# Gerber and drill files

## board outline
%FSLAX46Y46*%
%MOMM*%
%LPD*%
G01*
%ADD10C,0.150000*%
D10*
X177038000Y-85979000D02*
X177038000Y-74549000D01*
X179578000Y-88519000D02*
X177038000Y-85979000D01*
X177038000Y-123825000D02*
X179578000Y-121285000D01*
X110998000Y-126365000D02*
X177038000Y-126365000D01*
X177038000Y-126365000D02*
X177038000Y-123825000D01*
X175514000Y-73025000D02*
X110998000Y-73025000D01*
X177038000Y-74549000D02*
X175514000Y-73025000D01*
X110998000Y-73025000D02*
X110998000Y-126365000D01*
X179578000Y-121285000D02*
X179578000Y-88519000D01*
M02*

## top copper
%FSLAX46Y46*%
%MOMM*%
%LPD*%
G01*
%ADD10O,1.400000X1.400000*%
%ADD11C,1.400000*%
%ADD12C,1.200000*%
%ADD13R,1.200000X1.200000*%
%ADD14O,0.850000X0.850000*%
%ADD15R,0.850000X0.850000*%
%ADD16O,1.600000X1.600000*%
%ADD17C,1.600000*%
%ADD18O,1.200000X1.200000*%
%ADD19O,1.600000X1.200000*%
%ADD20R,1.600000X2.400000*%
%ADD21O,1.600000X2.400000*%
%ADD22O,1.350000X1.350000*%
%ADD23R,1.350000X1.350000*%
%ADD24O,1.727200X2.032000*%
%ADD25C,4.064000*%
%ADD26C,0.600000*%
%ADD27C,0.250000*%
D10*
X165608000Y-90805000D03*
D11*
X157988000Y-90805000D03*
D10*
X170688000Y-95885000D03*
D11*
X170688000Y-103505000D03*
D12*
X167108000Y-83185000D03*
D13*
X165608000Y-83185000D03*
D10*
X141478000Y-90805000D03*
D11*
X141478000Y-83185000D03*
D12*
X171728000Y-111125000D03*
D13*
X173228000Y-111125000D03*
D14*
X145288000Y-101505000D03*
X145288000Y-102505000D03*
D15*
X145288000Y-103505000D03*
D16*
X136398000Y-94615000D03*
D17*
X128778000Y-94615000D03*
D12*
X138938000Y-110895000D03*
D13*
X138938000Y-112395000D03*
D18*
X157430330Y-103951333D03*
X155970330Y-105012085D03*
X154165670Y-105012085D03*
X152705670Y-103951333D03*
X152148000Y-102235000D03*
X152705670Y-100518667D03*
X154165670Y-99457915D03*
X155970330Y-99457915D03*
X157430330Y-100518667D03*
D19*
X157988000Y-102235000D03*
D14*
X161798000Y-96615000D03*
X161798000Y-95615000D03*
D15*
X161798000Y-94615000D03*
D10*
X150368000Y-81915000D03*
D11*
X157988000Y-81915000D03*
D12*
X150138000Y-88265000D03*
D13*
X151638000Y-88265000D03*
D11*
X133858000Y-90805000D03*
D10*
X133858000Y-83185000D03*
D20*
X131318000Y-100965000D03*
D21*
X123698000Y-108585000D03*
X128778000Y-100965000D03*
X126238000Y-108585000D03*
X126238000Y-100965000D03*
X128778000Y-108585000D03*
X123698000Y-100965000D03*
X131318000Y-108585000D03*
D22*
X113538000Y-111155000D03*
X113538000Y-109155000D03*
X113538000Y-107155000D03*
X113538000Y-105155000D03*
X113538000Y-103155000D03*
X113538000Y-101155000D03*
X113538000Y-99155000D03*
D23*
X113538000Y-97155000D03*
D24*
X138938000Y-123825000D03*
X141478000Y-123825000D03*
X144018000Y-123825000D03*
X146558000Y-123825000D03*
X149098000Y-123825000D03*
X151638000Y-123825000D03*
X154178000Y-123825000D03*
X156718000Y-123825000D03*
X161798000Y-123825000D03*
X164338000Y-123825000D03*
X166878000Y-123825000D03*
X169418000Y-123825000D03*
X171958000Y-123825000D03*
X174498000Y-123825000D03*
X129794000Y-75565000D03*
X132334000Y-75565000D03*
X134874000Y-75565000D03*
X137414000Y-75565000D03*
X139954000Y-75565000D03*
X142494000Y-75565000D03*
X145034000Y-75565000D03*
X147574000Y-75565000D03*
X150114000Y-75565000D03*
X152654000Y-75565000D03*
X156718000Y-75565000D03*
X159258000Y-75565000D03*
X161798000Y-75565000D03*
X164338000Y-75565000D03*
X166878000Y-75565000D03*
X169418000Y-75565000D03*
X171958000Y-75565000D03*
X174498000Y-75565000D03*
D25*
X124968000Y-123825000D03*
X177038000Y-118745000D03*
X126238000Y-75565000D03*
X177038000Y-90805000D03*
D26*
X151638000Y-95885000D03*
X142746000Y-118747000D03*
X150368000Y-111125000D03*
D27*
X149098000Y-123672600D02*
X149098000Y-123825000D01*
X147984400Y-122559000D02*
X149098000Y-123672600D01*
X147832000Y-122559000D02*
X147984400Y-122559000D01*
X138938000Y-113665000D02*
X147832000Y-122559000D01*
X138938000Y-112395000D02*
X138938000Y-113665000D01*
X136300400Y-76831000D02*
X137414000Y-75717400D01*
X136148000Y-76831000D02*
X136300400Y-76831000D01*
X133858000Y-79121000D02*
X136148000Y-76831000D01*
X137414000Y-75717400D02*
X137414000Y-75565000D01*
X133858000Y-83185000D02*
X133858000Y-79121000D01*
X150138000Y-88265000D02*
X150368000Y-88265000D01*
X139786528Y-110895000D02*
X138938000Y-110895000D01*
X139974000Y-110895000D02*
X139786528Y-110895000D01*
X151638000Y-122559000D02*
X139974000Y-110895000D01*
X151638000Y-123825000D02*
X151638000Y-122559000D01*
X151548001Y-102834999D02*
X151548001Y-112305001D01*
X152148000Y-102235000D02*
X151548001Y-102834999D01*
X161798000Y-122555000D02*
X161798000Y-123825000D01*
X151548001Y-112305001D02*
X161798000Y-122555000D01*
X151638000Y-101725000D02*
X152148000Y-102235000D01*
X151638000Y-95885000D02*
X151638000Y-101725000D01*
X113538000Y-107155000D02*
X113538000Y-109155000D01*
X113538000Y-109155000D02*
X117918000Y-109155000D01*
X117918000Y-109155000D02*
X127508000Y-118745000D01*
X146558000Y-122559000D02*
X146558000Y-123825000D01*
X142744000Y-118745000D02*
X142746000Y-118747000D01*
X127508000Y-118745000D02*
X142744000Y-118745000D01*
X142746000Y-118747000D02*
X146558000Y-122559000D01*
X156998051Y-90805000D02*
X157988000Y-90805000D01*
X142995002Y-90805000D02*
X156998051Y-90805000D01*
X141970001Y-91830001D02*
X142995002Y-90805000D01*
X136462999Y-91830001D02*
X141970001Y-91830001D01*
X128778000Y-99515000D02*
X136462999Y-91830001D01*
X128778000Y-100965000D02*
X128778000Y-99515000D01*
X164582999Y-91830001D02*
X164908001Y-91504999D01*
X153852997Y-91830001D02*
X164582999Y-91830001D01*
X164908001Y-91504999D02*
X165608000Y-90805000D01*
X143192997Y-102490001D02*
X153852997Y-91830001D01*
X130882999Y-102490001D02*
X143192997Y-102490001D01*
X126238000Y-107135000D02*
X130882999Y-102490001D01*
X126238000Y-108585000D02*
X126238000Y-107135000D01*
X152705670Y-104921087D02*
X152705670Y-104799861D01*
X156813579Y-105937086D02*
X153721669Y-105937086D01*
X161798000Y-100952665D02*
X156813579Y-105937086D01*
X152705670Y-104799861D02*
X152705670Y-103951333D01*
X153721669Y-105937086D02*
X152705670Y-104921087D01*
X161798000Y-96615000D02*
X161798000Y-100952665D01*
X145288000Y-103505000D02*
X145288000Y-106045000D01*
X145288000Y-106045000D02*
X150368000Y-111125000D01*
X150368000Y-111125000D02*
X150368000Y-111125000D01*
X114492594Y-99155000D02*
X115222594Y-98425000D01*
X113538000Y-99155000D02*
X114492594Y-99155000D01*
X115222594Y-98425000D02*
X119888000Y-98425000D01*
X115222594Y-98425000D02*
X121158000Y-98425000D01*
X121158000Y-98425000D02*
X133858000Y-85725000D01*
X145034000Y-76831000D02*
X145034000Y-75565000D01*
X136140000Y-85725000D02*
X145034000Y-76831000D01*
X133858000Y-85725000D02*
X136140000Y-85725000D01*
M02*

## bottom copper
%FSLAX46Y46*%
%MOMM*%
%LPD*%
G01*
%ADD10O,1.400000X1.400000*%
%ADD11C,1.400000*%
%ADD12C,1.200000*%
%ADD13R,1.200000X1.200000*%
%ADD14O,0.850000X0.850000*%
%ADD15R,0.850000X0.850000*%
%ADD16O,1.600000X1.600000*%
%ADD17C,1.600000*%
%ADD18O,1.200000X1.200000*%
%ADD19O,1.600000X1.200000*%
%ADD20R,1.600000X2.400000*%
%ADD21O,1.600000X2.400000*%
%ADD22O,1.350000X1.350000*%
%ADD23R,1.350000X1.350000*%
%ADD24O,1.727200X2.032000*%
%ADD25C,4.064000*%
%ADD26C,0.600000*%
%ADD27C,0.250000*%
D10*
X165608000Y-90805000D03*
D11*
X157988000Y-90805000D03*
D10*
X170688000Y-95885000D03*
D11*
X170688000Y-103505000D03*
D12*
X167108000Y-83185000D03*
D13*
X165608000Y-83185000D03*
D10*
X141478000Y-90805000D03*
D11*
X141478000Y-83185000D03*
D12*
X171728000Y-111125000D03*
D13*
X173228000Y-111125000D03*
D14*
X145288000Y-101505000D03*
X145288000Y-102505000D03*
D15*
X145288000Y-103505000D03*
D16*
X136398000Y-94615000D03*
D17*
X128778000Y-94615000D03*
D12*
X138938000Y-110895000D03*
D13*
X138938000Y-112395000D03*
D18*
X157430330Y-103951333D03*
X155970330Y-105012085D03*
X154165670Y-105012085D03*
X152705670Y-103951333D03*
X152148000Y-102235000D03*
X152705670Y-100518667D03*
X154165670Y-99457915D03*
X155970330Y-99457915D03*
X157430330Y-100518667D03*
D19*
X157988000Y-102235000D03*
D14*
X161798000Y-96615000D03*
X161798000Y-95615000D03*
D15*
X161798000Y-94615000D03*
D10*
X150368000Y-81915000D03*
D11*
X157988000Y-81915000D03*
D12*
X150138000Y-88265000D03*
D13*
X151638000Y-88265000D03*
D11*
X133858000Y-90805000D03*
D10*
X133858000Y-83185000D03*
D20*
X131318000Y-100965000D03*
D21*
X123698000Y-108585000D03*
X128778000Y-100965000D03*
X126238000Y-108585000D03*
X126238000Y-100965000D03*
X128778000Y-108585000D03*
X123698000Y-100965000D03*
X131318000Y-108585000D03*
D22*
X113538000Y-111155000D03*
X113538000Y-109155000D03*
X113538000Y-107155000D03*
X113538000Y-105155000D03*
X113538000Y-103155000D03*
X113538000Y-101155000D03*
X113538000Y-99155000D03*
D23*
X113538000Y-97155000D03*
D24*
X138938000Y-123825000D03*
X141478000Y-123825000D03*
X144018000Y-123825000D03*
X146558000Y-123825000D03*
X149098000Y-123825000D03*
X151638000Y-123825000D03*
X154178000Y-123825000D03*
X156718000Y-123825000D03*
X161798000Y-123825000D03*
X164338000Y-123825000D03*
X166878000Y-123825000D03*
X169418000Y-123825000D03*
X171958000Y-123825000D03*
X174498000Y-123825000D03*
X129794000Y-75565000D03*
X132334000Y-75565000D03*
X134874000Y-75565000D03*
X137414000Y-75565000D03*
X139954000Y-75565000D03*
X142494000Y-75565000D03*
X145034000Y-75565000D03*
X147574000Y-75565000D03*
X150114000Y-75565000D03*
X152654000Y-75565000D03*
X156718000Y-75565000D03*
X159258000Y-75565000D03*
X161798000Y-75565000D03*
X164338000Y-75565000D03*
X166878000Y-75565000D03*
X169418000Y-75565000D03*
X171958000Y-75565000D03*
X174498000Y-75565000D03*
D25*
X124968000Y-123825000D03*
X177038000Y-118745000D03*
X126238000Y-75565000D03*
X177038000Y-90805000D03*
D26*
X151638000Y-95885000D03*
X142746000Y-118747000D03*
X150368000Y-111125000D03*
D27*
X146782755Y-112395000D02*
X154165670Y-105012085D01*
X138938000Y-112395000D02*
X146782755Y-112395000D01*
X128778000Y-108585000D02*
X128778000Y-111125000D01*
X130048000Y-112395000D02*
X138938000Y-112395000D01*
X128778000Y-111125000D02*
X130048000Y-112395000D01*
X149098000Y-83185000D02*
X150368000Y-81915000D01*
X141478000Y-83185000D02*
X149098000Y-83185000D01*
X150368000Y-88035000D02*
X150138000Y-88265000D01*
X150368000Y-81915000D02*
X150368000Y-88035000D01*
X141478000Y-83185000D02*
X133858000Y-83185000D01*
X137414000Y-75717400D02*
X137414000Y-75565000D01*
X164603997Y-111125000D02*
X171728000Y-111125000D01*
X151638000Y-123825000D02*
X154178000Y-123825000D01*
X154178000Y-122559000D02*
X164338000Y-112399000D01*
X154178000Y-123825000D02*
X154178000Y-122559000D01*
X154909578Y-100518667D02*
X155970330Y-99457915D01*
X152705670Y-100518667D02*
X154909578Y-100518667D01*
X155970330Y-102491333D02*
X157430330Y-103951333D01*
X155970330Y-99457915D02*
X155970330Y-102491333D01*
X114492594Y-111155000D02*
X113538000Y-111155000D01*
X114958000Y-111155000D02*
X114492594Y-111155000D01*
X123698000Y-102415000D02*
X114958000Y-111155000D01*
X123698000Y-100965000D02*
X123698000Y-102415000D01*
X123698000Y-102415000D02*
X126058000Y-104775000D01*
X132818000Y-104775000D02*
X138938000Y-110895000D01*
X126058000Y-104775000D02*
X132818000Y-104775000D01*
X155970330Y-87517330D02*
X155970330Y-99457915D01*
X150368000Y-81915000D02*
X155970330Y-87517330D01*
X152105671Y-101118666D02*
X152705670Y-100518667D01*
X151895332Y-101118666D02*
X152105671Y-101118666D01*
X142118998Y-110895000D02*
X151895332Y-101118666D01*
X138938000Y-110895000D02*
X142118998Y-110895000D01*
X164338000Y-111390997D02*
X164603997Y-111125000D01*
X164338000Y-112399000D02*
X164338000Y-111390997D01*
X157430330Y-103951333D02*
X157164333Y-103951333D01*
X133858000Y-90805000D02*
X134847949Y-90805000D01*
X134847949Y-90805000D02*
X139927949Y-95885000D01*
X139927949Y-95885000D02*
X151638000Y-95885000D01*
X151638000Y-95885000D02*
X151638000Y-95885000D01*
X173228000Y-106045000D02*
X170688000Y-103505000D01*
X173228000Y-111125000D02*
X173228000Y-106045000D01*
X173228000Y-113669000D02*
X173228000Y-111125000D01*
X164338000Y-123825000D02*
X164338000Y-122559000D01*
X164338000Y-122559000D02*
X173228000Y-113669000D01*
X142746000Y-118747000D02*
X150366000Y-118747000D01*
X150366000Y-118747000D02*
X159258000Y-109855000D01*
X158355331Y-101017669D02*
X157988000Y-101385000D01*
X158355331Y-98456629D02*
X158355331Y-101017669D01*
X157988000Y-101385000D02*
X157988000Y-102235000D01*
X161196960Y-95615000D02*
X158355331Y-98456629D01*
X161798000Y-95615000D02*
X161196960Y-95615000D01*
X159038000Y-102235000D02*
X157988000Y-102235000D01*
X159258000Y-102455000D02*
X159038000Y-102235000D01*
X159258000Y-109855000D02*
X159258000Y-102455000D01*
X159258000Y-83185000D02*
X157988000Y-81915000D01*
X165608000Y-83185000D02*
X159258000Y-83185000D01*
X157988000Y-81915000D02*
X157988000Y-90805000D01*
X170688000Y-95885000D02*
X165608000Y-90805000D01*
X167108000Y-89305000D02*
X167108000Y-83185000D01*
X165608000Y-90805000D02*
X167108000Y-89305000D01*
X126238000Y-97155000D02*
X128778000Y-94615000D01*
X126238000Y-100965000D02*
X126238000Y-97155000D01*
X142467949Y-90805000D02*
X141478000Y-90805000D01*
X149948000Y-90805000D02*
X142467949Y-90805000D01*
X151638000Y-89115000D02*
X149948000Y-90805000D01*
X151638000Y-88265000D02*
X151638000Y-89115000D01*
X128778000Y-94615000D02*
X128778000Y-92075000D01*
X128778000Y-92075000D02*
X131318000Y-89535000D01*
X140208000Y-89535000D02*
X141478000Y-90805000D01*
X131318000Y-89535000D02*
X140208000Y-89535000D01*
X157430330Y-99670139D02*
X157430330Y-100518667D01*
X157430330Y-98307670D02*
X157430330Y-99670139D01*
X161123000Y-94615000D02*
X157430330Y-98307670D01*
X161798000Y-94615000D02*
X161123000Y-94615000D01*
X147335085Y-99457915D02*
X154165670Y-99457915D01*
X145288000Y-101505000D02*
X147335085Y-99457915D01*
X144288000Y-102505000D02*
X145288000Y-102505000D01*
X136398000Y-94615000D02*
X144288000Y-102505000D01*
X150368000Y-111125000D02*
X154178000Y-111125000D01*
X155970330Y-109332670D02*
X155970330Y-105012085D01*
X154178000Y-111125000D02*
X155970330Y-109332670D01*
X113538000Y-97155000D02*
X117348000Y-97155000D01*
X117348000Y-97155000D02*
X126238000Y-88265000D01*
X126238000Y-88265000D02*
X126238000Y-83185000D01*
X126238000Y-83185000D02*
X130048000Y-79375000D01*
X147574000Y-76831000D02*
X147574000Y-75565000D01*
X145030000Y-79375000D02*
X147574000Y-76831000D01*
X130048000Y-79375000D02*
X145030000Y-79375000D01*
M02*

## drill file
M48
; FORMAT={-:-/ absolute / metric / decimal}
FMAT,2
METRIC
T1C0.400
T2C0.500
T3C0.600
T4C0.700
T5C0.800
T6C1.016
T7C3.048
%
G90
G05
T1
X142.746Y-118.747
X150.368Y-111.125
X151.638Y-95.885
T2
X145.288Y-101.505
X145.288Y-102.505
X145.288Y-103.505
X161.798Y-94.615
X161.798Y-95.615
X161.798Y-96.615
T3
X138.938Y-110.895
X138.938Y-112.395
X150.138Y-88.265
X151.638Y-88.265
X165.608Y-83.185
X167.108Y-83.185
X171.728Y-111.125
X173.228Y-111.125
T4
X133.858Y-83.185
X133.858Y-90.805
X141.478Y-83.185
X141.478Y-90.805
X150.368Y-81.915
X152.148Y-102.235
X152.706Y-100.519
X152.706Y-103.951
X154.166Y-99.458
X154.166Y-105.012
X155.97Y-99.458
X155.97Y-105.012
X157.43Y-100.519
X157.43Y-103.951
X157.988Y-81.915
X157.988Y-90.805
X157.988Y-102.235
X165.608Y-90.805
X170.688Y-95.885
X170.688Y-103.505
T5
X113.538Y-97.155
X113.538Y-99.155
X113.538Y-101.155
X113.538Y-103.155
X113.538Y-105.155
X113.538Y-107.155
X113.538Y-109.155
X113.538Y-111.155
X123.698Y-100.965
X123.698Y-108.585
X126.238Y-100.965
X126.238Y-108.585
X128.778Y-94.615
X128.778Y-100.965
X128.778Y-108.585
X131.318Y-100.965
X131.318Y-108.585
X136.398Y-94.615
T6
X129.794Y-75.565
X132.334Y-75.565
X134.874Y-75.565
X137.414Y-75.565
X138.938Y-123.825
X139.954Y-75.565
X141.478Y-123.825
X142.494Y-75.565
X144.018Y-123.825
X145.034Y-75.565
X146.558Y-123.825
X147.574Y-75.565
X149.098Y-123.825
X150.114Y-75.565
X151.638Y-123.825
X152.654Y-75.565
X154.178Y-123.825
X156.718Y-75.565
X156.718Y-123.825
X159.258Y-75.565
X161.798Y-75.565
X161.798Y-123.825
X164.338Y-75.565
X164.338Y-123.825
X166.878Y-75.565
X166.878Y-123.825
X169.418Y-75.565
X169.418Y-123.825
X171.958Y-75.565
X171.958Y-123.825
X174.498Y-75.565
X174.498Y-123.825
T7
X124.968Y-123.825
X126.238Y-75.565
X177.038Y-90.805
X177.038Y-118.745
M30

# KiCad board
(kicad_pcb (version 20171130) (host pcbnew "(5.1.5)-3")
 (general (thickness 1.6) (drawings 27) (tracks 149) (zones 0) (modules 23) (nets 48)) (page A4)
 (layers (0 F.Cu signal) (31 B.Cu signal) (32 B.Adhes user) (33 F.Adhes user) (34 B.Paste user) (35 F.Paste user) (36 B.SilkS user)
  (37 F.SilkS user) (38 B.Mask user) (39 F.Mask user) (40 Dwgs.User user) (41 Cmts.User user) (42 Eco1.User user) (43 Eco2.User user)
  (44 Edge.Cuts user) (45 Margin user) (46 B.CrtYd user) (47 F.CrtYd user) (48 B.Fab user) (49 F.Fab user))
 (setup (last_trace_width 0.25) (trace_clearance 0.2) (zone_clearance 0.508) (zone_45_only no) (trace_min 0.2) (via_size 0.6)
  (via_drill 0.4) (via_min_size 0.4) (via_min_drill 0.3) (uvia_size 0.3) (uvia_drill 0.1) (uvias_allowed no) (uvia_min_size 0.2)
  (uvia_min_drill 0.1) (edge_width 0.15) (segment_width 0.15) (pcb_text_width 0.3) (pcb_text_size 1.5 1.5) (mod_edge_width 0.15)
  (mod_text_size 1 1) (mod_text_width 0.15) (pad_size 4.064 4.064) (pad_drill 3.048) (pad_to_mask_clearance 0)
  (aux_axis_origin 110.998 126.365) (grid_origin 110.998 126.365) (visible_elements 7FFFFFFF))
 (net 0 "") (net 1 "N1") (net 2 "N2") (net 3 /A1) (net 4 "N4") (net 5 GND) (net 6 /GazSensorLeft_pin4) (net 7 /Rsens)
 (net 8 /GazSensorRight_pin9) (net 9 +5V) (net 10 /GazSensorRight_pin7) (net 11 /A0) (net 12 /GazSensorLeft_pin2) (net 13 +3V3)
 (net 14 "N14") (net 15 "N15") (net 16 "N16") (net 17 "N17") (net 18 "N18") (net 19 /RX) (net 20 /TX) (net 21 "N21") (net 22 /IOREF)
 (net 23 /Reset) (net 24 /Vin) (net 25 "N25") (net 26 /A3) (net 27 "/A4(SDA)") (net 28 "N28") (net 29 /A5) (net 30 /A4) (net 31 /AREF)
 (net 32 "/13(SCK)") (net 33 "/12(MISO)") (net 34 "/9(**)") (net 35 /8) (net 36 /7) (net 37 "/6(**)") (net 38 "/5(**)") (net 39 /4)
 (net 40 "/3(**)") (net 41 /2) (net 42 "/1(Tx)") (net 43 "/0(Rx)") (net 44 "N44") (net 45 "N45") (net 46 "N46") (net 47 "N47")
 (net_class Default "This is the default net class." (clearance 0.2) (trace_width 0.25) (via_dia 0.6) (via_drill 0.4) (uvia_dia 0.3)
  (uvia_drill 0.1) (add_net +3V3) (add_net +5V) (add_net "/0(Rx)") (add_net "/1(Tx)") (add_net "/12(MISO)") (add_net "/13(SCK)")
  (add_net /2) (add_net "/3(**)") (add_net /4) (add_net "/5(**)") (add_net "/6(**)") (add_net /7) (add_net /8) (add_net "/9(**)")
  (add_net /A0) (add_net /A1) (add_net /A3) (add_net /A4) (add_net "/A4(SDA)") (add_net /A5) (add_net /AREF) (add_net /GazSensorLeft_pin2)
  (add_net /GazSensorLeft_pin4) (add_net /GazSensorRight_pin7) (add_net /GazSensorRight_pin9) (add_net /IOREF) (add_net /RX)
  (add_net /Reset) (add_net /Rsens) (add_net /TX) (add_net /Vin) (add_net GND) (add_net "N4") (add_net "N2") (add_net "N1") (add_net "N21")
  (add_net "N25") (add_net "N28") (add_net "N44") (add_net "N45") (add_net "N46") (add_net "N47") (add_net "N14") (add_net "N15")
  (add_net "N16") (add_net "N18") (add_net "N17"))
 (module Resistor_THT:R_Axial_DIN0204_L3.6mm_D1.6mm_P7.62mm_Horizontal (layer F.Cu) (at 157.988 90.805)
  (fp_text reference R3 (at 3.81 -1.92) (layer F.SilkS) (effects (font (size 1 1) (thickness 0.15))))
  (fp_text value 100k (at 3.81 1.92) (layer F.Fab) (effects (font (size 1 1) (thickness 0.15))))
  (pad 2 thru_hole oval (at 7.62 0) (size 1.4 1.4) (drill 0.7) (layers *.Cu *.Mask) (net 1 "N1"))
  (pad 1 thru_hole circle (at 0 0) (size 1.4 1.4) (drill 0.7) (layers *.Cu *.Mask) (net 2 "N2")))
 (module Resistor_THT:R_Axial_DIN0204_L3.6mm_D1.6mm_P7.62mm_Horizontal (layer F.Cu) (at 170.688 103.505 90)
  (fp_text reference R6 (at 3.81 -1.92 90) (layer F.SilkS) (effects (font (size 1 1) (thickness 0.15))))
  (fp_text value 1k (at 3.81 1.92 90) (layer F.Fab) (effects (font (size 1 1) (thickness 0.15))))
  (pad 2 thru_hole oval (at 7.62 0 90) (size 1.4 1.4) (drill 0.7) (layers *.Cu *.Mask) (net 1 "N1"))
  (pad 1 thru_hole circle (at 0 0 90) (size 1.4 1.4) (drill 0.7) (layers *.Cu *.Mask) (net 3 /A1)))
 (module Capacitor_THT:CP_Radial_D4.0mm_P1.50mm (layer F.Cu) (at 165.608 83.185)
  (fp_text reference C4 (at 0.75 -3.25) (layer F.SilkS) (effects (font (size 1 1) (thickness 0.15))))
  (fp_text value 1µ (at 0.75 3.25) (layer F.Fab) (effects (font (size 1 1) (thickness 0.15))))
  (pad 2 thru_hole circle (at 1.5 0) (size 1.2 1.2) (drill 0.6) (layers *.Cu *.Mask) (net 1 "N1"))
  (pad 1 thru_hole rect (at 0 0) (size 1.2 1.2) (drill 0.6) (layers *.Cu *.Mask) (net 2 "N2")))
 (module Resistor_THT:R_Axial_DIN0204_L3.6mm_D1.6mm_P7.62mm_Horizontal (layer F.Cu) (at 141.478 83.185 270)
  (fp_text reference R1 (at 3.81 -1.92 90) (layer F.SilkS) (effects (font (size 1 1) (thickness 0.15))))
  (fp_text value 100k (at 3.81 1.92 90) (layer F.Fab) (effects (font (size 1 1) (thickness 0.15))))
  (pad 2 thru_hole oval (at 7.62 0 270) (size 1.4 1.4) (drill 0.7) (layers *.Cu *.Mask) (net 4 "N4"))
  (pad 1 thru_hole circle (at 0 0 270) (size 1.4 1.4) (drill 0.7) (layers *.Cu *.Mask) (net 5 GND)))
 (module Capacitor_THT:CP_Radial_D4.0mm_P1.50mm (layer F.Cu) (at 173.228 111.125 180)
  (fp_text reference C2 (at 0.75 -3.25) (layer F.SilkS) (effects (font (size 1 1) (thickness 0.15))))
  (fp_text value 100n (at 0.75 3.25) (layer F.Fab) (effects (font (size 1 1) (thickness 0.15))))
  (pad 2 thru_hole circle (at 1.5 0 180) (size 1.2 1.2) (drill 0.6) (layers *.Cu *.Mask) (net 5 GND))
  (pad 1 thru_hole rect (at 0 0 180) (size 1.2 1.2) (drill 0.6) (layers *.Cu *.Mask) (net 3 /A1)))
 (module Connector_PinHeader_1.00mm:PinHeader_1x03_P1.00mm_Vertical (layer F.Cu) (at 145.288 103.505 180)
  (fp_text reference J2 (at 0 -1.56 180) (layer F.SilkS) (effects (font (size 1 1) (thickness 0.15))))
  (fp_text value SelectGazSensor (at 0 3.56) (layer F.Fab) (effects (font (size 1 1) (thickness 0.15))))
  (pad 3 thru_hole oval (at 0 2 180) (size 0.85 0.85) (drill 0.5) (layers *.Cu *.Mask) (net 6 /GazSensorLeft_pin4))
  (pad 2 thru_hole oval (at 0 1 180) (size 0.85 0.85) (drill 0.5) (layers *.Cu *.Mask) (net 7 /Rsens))
  (pad 1 thru_hole rect (at 0 0 180) (size 0.85 0.85) (drill 0.5) (layers *.Cu *.Mask) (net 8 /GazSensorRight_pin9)))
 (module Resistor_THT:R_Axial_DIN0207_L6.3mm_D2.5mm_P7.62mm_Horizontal (layer F.Cu) (at 128.778 94.615)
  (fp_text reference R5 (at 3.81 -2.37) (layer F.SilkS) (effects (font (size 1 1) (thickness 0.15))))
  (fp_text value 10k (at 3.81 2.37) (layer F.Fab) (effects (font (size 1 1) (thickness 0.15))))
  (pad 2 thru_hole oval (at 7.62 0) (size 1.6 1.6) (drill 0.8) (layers *.Cu *.Mask) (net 7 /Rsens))
  (pad 1 thru_hole circle (at 0 0) (size 1.6 1.6) (drill 0.8) (layers *.Cu *.Mask) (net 4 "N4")))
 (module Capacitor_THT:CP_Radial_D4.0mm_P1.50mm (layer F.Cu) (at 138.938 112.395 90)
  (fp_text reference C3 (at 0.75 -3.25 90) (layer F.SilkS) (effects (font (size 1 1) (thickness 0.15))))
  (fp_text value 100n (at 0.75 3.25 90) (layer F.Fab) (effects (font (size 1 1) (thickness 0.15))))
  (pad 2 thru_hole circle (at 1.5 0 90) (size 1.2 1.2) (drill 0.6) (layers *.Cu *.Mask) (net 5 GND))
  (pad 1 thru_hole rect (at 0 0 90) (size 1.2 1.2) (drill 0.6) (layers *.Cu *.Mask) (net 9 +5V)))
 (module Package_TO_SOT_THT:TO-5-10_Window (layer F.Cu) (at 157.988 102.235 180)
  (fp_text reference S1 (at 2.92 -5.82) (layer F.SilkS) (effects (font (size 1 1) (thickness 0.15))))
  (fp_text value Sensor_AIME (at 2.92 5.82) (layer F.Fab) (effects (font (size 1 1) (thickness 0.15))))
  (pad 10 thru_hole oval (at 0.55767 -1.716333 180) (size 1.2 1.2) (drill 0.7) (layers *.Cu *.Mask) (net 5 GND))
  (pad 9 thru_hole oval (at 2.01767 -2.777085 180) (size 1.2 1.2) (drill 0.7) (layers *.Cu *.Mask) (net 8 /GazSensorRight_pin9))
  (pad 8 thru_hole oval (at 3.82233 -2.777085 180) (size 1.2 1.2) (drill 0.7) (layers *.Cu *.Mask) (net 9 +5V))
  (pad 7 thru_hole oval (at 5.28233 -1.716333 180) (size 1.2 1.2) (drill 0.7) (layers *.Cu *.Mask) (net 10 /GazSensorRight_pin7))
  (pad 6 thru_hole oval (at 5.84 0 180) (size 1.2 1.2) (drill 0.7) (layers *.Cu *.Mask) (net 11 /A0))
  (pad 5 thru_hole oval (at 5.28233 1.716333 180) (size 1.2 1.2) (drill 0.7) (layers *.Cu *.Mask) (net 5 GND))
  (pad 4 thru_hole oval (at 3.82233 2.777085 180) (size 1.2 1.2) (drill 0.7) (layers *.Cu *.Mask) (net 6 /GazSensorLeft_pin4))
  (pad 3 thru_hole oval (at 2.01767 2.777085 180) (size 1.2 1.2) (drill 0.7) (layers *.Cu *.Mask) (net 5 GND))
  (pad 2 thru_hole oval (at 0.55767 1.716333 180) (size 1.2 1.2) (drill 0.7) (layers *.Cu *.Mask) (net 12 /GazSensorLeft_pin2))
  (pad 1 thru_hole oval (at 0 0 180) (size 1.6 1.2) (drill 0.7) (layers *.Cu *.Mask) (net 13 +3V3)))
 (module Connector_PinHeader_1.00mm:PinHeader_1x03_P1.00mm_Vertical (layer F.Cu) (at 161.798 94.615)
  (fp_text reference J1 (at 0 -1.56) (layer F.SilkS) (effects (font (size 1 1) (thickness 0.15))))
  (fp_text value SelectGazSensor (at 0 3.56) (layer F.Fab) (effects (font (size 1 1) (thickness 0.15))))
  (pad 3 thru_hole oval (at 0 2) (size 0.85 0.85) (drill 0.5) (layers *.Cu *.Mask) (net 10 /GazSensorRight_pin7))
  (pad 2 thru_hole oval (at 0 1) (size 0.85 0.85) (drill 0.5) (layers *.Cu *.Mask) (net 13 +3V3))
  (pad 1 thru_hole rect (at 0 0) (size 0.85 0.85) (drill 0.5) (layers *.Cu *.Mask) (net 12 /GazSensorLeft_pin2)))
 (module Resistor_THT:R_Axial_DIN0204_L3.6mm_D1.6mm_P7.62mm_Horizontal (layer F.Cu) (at 157.988 81.915 180)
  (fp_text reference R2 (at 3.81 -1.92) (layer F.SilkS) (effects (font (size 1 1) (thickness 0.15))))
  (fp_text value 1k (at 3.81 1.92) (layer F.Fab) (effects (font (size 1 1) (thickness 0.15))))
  (pad 2 thru_hole oval (at 7.62 0 180) (size 1.4 1.4) (drill 0.7) (layers *.Cu *.Mask) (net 5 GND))
  (pad 1 thru_hole circle (at 0 0 180) (size 1.4 1.4) (drill 0.7) (layers *.Cu *.Mask) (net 2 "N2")))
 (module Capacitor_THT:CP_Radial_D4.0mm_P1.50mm (layer F.Cu) (at 151.638 88.265 180)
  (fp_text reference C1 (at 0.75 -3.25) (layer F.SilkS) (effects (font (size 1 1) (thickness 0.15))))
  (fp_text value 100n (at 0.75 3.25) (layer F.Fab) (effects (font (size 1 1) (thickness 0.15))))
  (pad 2 thru_hole circle (at 1.5 0 180) (size 1.2 1.2) (drill 0.6) (layers *.Cu *.Mask) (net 5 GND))
  (pad 1 thru_hole rect (at 0 0 180) (size 1.2 1.2) (drill 0.6) (layers *.Cu *.Mask) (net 4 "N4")))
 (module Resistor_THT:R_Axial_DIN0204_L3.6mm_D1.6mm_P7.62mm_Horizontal (layer F.Cu) (at 133.858 90.805 90)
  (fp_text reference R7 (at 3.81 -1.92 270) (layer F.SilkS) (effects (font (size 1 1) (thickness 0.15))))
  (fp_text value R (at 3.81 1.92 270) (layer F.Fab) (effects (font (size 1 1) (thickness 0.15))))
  (pad 1 thru_hole circle (at 0 0 90) (size 1.4 1.4) (drill 0.7) (layers *.Cu *.Mask) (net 11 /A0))
  (pad 2 thru_hole oval (at 7.62 0 90) (size 1.4 1.4) (drill 0.7) (layers *.Cu *.Mask) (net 5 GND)))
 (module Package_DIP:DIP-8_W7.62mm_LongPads (layer F.Cu) (at 131.318 100.965 270)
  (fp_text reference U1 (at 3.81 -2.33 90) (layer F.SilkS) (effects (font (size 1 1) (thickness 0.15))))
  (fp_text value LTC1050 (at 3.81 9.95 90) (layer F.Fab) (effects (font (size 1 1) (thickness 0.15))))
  (pad 1 thru_hole rect (at 0 0 270) (size 2.4 1.6) (drill 0.8) (layers *.Cu *.Mask) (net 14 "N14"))
  (pad 5 thru_hole oval (at 7.62 7.62 270) (size 2.4 1.6) (drill 0.8) (layers *.Cu *.Mask) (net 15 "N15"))
  (pad 2 thru_hole oval (at 0 2.54 270) (size 2.4 1.6) (drill 0.8) (layers *.Cu *.Mask) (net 2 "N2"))
  (pad 6 thru_hole oval (at 7.62 5.08 270) (size 2.4 1.6) (drill 0.8) (layers *.Cu *.Mask) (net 1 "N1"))
  (pad 3 thru_hole oval (at 0 5.08 270) (size 2.4 1.6) (drill 0.8) (layers *.Cu *.Mask) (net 4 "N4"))
  (pad 7 thru_hole oval (at 7.62 2.54 270) (size 2.4 1.6) (drill 0.8) (layers *.Cu *.Mask) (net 9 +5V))
  (pad 4 thru_hole oval (at 0 7.62 270) (size 2.4 1.6) (drill 0.8) (layers *.Cu *.Mask) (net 5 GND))
  (pad 8 thru_hole oval (at 7.62 0 270) (size 2.4 1.6) (drill 0.8) (layers *.Cu *.Mask) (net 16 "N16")))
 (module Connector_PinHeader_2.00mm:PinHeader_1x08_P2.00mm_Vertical (layer F.Cu) (at 113.538 97.155)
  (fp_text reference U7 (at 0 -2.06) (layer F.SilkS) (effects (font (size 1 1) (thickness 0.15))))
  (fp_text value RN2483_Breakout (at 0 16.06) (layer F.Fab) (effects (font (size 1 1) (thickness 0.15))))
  (pad 8 thru_hole oval (at 0 14) (size 1.35 1.35) (drill 0.8) (layers *.Cu *.Mask) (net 5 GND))
  (pad 7 thru_hole oval (at 0 12) (size 1.35 1.35) (drill 0.8) (layers *.Cu *.Mask) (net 13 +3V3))
  (pad 6 thru_hole oval (at 0 10) (size 1.35 1.35) (drill 0.8) (layers *.Cu *.Mask) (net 13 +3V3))
  (pad 5 thru_hole oval (at 0 8) (size 1.35 1.35) (drill 0.8) (layers *.Cu *.Mask))
  (pad 4 thru_hole oval (at 0 6) (size 1.35 1.35) (drill 0.8) (layers *.Cu *.Mask) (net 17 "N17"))
  (pad 3 thru_hole oval (at 0 4) (size 1.35 1.35) (drill 0.8) (layers *.Cu *.Mask) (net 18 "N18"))
  (pad 2 thru_hole oval (at 0 2) (size 1.35 1.35) (drill 0.8) (layers *.Cu *.Mask) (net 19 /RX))
  (pad 1 thru_hole rect (at 0 0) (size 1.35 1.35) (drill 0.8) (layers *.Cu *.Mask) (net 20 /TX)))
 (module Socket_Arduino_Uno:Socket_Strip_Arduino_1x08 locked (layer F.Cu) (at 138.938 123.825)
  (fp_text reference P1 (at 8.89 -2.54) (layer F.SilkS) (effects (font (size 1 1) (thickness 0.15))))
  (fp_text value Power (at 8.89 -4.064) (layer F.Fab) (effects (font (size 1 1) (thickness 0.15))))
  (pad 1 thru_hole oval (at 0 0) (size 1.7272 2.032) (drill 1.016) (layers *.Cu *.Mask F.SilkS) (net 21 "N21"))
  (pad 2 thru_hole oval (at 2.54 0) (size 1.7272 2.032) (drill 1.016) (layers *.Cu *.Mask F.SilkS) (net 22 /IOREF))
  (pad 3 thru_hole oval (at 5.08 0) (size 1.7272 2.032) (drill 1.016) (layers *.Cu *.Mask F.SilkS) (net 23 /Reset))
  (pad 4 thru_hole oval (at 7.62 0) (size 1.7272 2.032) (drill 1.016) (layers *.Cu *.Mask F.SilkS) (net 13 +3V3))
  (pad 5 thru_hole oval (at 10.16 0) (size 1.7272 2.032) (drill 1.016) (layers *.Cu *.Mask F.SilkS) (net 9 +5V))
  (pad 6 thru_hole oval (at 12.7 0) (size 1.7272 2.032) (drill 1.016) (layers *.Cu *.Mask F.SilkS) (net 5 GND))
  (pad 7 thru_hole oval (at 15.24 0) (size 1.7272 2.032) (drill 1.016) (layers *.Cu *.Mask F.SilkS) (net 5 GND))
  (pad 8 thru_hole oval (at 17.78 0) (size 1.7272 2.032) (drill 1.016) (layers *.Cu *.Mask F.SilkS) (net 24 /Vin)))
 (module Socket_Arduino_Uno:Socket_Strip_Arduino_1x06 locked (layer F.Cu) (at 161.798 123.825)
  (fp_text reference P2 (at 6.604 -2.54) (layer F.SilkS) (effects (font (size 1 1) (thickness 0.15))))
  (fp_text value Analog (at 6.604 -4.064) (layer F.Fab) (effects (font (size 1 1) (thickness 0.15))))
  (pad 1 thru_hole oval (at 0 0) (size 1.7272 2.032) (drill 1.016) (layers *.Cu *.Mask F.SilkS) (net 11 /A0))
  (pad 2 thru_hole oval (at 2.54 0) (size 1.7272 2.032) (drill 1.016) (layers *.Cu *.Mask F.SilkS) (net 3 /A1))
  (pad 3 thru_hole oval (at 5.08 0) (size 1.7272 2.032) (drill 1.016) (layers *.Cu *.Mask F.SilkS) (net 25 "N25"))
  (pad 4 thru_hole oval (at 7.62 0) (size 1.7272 2.032) (drill 1.016) (layers *.Cu *.Mask F.SilkS) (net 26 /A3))
  (pad 5 thru_hole oval (at 10.16 0) (size 1.7272 2.032) (drill 1.016) (layers *.Cu *.Mask F.SilkS) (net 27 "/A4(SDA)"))
  (pad 6 thru_hole oval (at 12.7 0) (size 1.7272 2.032) (drill 1.016) (layers *.Cu *.Mask F.SilkS) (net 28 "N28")))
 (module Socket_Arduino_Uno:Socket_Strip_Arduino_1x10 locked (layer F.Cu) (at 129.794 75.565)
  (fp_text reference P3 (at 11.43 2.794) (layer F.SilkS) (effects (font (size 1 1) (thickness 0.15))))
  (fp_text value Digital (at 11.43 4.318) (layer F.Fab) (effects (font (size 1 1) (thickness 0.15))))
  (pad 1 thru_hole oval (at 0 0) (size 1.7272 2.032) (drill 1.016) (layers *.Cu *.Mask F.SilkS) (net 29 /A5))
  (pad 2 thru_hole oval (at 2.54 0) (size 1.7272 2.032) (drill 1.016) (layers *.Cu *.Mask F.SilkS) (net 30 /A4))
  (pad 3 thru_hole oval (at 5.08 0) (size 1.7272 2.032) (drill 1.016) (layers *.Cu *.Mask F.SilkS) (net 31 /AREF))
  (pad 4 thru_hole oval (at 7.62 0) (size 1.7272 2.032) (drill 1.016) (layers *.Cu *.Mask F.SilkS) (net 5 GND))
  (pad 5 thru_hole oval (at 10.16 0) (size 1.7272 2.032) (drill 1.016) (layers *.Cu *.Mask F.SilkS) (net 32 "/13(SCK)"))
  (pad 6 thru_hole oval (at 12.7 0) (size 1.7272 2.032) (drill 1.016) (layers *.Cu *.Mask F.SilkS) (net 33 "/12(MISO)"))
  (pad 7 thru_hole oval (at 15.24 0) (size 1.7272 2.032) (drill 1.016) (layers *.Cu *.Mask F.SilkS) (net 19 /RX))
  (pad 8 thru_hole oval (at 17.78 0) (size 1.7272 2.032) (drill 1.016) (layers *.Cu *.Mask F.SilkS) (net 20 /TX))
  (pad 9 thru_hole oval (at 20.32 0) (size 1.7272 2.032) (drill 1.016) (layers *.Cu *.Mask F.SilkS) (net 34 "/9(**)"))
  (pad 10 thru_hole oval (at 22.86 0) (size 1.7272 2.032) (drill 1.016) (layers *.Cu *.Mask F.SilkS) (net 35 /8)))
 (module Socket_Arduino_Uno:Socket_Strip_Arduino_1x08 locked (layer F.Cu) (at 156.718 75.565)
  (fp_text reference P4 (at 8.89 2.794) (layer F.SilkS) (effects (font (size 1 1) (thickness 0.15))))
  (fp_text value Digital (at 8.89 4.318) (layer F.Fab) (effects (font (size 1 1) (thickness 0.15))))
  (pad 1 thru_hole oval (at 0 0) (size 1.7272 2.032) (drill 1.016) (layers *.Cu *.Mask F.SilkS) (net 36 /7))
  (pad 2 thru_hole oval (at 2.54 0) (size 1.7272 2.032) (drill 1.016) (layers *.Cu *.Mask F.SilkS) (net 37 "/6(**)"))
  (pad 3 thru_hole oval (at 5.08 0) (size 1.7272 2.032) (drill 1.016) (layers *.Cu *.Mask F.SilkS) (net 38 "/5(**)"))
  (pad 4 thru_hole oval (at 7.62 0) (size 1.7272 2.032) (drill 1.016) (layers *.Cu *.Mask F.SilkS) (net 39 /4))
  (pad 5 thru_hole oval (at 10.16 0) (size 1.7272 2.032) (drill 1.016) (layers *.Cu *.Mask F.SilkS) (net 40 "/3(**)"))
  (pad 6 thru_hole oval (at 12.7 0) (size 1.7272 2.032) (drill 1.016) (layers *.Cu *.Mask F.SilkS) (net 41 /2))
  (pad 7 thru_hole oval (at 15.24 0) (size 1.7272 2.032) (drill 1.016) (layers *.Cu *.Mask F.SilkS) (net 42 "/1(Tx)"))
  (pad 8 thru_hole oval (at 17.78 0) (size 1.7272 2.032) (drill 1.016) (layers *.Cu *.Mask F.SilkS) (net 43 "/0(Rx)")))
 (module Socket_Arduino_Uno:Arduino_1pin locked (layer F.Cu) (at 124.968 123.825)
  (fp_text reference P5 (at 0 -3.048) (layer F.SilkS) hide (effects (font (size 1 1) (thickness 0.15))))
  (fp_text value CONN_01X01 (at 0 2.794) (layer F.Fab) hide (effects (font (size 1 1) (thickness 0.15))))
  (pad 1 thru_hole circle (at 0 0) (size 4.064 4.064) (drill 3.048) (layers *.Cu *.Mask F.SilkS) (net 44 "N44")))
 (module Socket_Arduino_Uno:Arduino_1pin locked (layer F.Cu) (at 177.038 118.745)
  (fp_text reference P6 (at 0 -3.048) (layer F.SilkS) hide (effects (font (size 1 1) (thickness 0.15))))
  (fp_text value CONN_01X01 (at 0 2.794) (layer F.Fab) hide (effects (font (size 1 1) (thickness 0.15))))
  (pad 1 thru_hole circle (at 0 0) (size 4.064 4.064) (drill 3.048) (layers *.Cu *.Mask F.SilkS) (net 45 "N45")))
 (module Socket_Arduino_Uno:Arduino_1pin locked (layer F.Cu) (at 126.238 75.565)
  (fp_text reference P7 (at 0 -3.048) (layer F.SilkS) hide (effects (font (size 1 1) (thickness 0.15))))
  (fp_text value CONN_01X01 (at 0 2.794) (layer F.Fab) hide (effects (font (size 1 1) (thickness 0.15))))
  (pad 1 thru_hole circle (at 0 0) (size 4.064 4.064) (drill 3.048) (layers *.Cu *.Mask F.SilkS) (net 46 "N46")))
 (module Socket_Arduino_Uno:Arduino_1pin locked (layer F.Cu) (at 177.038 90.805)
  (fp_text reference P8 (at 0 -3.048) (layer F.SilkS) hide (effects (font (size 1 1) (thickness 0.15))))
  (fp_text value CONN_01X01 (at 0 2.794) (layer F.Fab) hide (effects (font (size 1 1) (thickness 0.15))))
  (pad 1 thru_hole circle (at 0 0) (size 4.064 4.064) (drill 3.048) (layers *.Cu *.Mask F.SilkS) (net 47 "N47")))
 (gr_line (start 177.038 85.979) (end 177.038 74.549) (angle 90) (layer Edge.Cuts) (width 0.15))
 (gr_line (start 179.578 88.519) (end 177.038 85.979) (angle 90) (layer Edge.Cuts) (width 0.15))
 (gr_line (start 177.038 123.825) (end 179.578 121.285) (angle 90) (layer Edge.Cuts) (width 0.15))
 (gr_line (start 110.998 126.365) (end 177.038 126.365) (angle 90) (layer Edge.Cuts) (width 0.15))
 (gr_line (start 177.038 126.365) (end 177.038 123.825) (angle 90) (layer Edge.Cuts) (width 0.15))
 (gr_line (start 175.514 73.025) (end 110.998 73.025) (angle 90) (layer Edge.Cuts) (width 0.15))
 (gr_line (start 177.038 74.549) (end 175.514 73.025) (angle 90) (layer Edge.Cuts) (width 0.15))
 (gr_line (start 110.998 73.025) (end 110.998 126.365) (angle 90) (layer Edge.Cuts) (width 0.15))
 (gr_line (start 179.578 121.285) (end 179.578 88.519) (angle 90) (layer Edge.Cuts) (width 0.15))
 (segment (start 149.098 123.6726) (end 149.098 123.825) (width 0.25) (layer F.Cu) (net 9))
 (segment (start 147.9844 122.559) (end 149.098 123.6726) (width 0.25) (layer F.Cu) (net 9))
 (segment (start 147.832 122.559) (end 147.9844 122.559) (width 0.25) (layer F.Cu) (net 9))
 (segment (start 138.938 113.665) (end 147.832 122.559) (width 0.25) (layer F.Cu) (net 9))
 (segment (start 138.938 112.395) (end 138.938 113.665) (width 0.25) (layer F.Cu) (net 9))
 (segment (start 146.782755 112.395) (end 154.16567 105.012085) (width 0.25) (layer B.Cu) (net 9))
 (segment (start 138.938 112.395) (end 146.782755 112.395) (width 0.25) (layer B.Cu) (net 9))
 (segment (start 128.778 108.585) (end 128.778 111.125) (width 0.25) (layer B.Cu) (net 9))
 (segment (start 130.048 112.395) (end 138.938 112.395) (width 0.25) (layer B.Cu) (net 9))
 (segment (start 128.778 111.125) (end 130.048 112.395) (width 0.25) (layer B.Cu) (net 9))
 (segment (start 149.098 83.185) (end 150.368 81.915) (width 0.25) (layer B.Cu) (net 5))
 (segment (start 141.478 83.185) (end 149.098 83.185) (width 0.25) (layer B.Cu) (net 5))
 (segment (start 150.368 88.035) (end 150.138 88.265) (width 0.25) (layer B.Cu) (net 5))
 (segment (start 150.368 81.915) (end 150.368 88.035) (width 0.25) (layer B.Cu) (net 5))
 (segment (start 141.478 83.185) (end 133.858 83.185) (width 0.25) (layer B.Cu) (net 5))
 (segment (start 137.414 75.7174) (end 137.414 75.565) (width 0.25) (layer B.Cu) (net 5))
 (segment (start 164.603997 111.125) (end 171.728 111.125) (width 0.25) (layer B.Cu) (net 5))
 (segment (start 151.638 123.825) (end 154.178 123.825) (width 0.25) (layer B.Cu) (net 5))
 (segment (start 154.178 122.559) (end 164.338 112.399) (width 0.25) (layer B.Cu) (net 5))
 (segment (start 154.178 123.825) (end 154.178 122.559) (width 0.25) (layer B.Cu) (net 5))
 (segment (start 154.909578 100.518667) (end 155.97033 99.457915) (width 0.25) (layer B.Cu) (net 5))
 (segment (start 152.70567 100.518667) (end 154.909578 100.518667) (width 0.25) (layer B.Cu) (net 5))
 (segment (start 155.97033 102.491333) (end 157.43033 103.951333) (width 0.25) (layer B.Cu) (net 5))
 (segment (start 155.97033 99.457915) (end 155.97033 102.491333) (width 0.25) (layer B.Cu) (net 5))
 (segment (start 114.492594 111.155) (end 113.538 111.155) (width 0.25) (layer B.Cu) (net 5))
 (segment (start 114.958 111.155) (end 114.492594 111.155) (width 0.25) (layer B.Cu) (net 5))
 (segment (start 123.698 102.415) (end 114.958 111.155) (width 0.25) (layer B.Cu) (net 5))
 (segment (start 123.698 100.965) (end 123.698 102.415) (width 0.25) (layer B.Cu) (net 5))
 (segment (start 123.698 102.415) (end 126.058 104.775) (width 0.25) (layer B.Cu) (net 5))
 (segment (start 132.818 104.775) (end 138.938 110.895) (width 0.25) (layer B.Cu) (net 5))
 (segment (start 126.058 104.775) (end 132.818 104.775) (width 0.25) (layer B.Cu) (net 5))
 (segment (start 136.3004 76.831) (end 137.414 75.7174) (width 0.25) (layer F.Cu) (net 5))
 (segment (start 136.148 76.831) (end 136.3004 76.831) (width 0.25) (layer F.Cu) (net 5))
 (segment (start 133.858 79.121) (end 136.148 76.831) (width 0.25) (layer F.Cu) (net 5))
 (segment (start 137.414 75.7174) (end 137.414 75.565) (width 0.25) (layer F.Cu) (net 5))
 (segment (start 133.858 83.185) (end 133.858 79.121) (width 0.25) (layer F.Cu) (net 5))
 (segment (start 150.138 88.265) (end 150.368 88.265) (width 0.25) (layer F.Cu) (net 5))
 (segment (start 155.97033 87.51733) (end 155.97033 99.457915) (width 0.25) (layer B.Cu) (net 5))
 (segment (start 150.368 81.915) (end 155.97033 87.51733) (width 0.25) (layer B.Cu) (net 5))
 (segment (start 152.105671 101.118666) (end 152.70567 100.518667) (width 0.25) (layer B.Cu) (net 5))
 (segment (start 151.895332 101.118666) (end 152.105671 101.118666) (width 0.25) (layer B.Cu) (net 5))
 (segment (start 142.118998 110.895) (end 151.895332 101.118666) (width 0.25) (layer B.Cu) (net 5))
 (segment (start 138.938 110.895) (end 142.118998 110.895) (width 0.25) (layer B.Cu) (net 5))
 (segment (start 164.338 111.390997) (end 164.603997 111.125) (width 0.25) (layer B.Cu) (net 5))
 (segment (start 164.338 112.399) (end 164.338 111.390997) (width 0.25) (layer B.Cu) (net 5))
 (segment (start 157.43033 103.951333) (end 157.164333 103.951333) (width 0.25) (layer B.Cu) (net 5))
 (segment (start 139.786528 110.895) (end 138.938 110.895) (width 0.25) (layer F.Cu) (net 5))
 (segment (start 139.974 110.895) (end 139.786528 110.895) (width 0.25) (layer F.Cu) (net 5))
 (segment (start 151.638 122.559) (end 139.974 110.895) (width 0.25) (layer F.Cu) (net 5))
 (segment (start 151.638 123.825) (end 151.638 122.559) (width 0.25) (layer F.Cu) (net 5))
 (segment (start 133.858 90.805) (end 134.847949 90.805) (width 0.25) (layer B.Cu) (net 11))
 (segment (start 151.548001 102.834999) (end 151.548001 112.305001) (width 0.25) (layer F.Cu) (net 11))
 (segment (start 152.148 102.235) (end 151.548001 102.834999) (width 0.25) (layer F.Cu) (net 11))
 (segment (start 161.798 122.555) (end 161.798 123.825) (width 0.25) (layer F.Cu) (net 11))
 (segment (start 151.548001 112.305001) (end 161.798 122.555) (width 0.25) (layer F.Cu) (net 11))
 (segment (start 134.847949 90.805) (end 139.927949 95.885) (width 0.25) (layer B.Cu) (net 11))
 (segment (start 139.927949 95.885) (end 151.638 95.885) (width 0.25) (layer B.Cu) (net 11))
 (segment (start 151.638 95.885) (end 151.638 95.885) (width 0.25) (layer B.Cu) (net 11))
 (via (at 151.638 95.885) (size 0.6) (drill 0.4) (layers F.Cu B.Cu) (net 11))
 (segment (start 151.638 101.725) (end 152.148 102.235) (width 0.25) (layer F.Cu) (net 11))
 (segment (start 151.638 95.885) (end 151.638 101.725) (width 0.25) (layer F.Cu) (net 11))
 (segment (start 173.228 106.045) (end 170.688 103.505) (width 0.25) (layer B.Cu) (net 3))
 (segment (start 173.228 111.125) (end 173.228 106.045) (width 0.25) (layer B.Cu) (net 3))
 (segment (start 173.228 113.669) (end 173.228 111.125) (width 0.25) (layer B.Cu) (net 3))
 (segment (start 164.338 123.825) (end 164.338 122.559) (width 0.25) (layer B.Cu) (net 3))
 (segment (start 164.338 122.559) (end 173.228 113.669) (width 0.25) (layer B.Cu) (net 3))
 (segment (start 113.538 107.155) (end 113.538 109.155) (width 0.25) (layer F.Cu) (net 13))
 (segment (start 113.538 109.155) (end 117.918 109.155) (width 0.25) (layer F.Cu) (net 13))
 (segment (start 117.918 109.155) (end 127.508 118.745) (width 0.25) (layer F.Cu) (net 13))
 (segment (start 146.558 122.559) (end 146.558 123.825) (width 0.25) (layer F.Cu) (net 13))
 (segment (start 142.744 118.745) (end 142.746 118.747) (width 0.25) (layer F.Cu) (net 13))
 (segment (start 127.508 118.745) (end 142.744 118.745) (width 0.25) (layer F.Cu) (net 13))
 (segment (start 142.746 118.747) (end 146.558 122.559) (width 0.25) (layer F.Cu) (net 13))
 (via (at 142.746 118.747) (size 0.6) (drill 0.4) (layers F.Cu B.Cu) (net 13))
 (segment (start 142.746 118.747) (end 150.366 118.747) (width 0.25) (layer B.Cu) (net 13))
 (segment (start 150.366 118.747) (end 159.258 109.855) (width 0.25) (layer B.Cu) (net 13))
 (segment (start 158.355331 101.017669) (end 157.988 101.385) (width 0.25) (layer B.Cu) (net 13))
 (segment (start 158.355331 98.456629) (end 158.355331 101.017669) (width 0.25) (layer B.Cu) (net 13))
 (segment (start 157.988 101.385) (end 157.988 102.235) (width 0.25) (layer B.Cu) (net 13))
 (segment (start 161.19696 95.615) (end 158.355331 98.456629) (width 0.25) (layer B.Cu) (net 13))
 (segment (start 161.798 95.615) (end 161.19696 95.615) (width 0.25) (layer B.Cu) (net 13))
 (segment (start 159.038 102.235) (end 157.988 102.235) (width 0.25) (layer B.Cu) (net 13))
 (segment (start 159.258 102.455) (end 159.038 102.235) (width 0.25) (layer B.Cu) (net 13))
 (segment (start 159.258 109.855) (end 159.258 102.455) (width 0.25) (layer B.Cu) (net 13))
 (segment (start 159.258 83.185) (end 157.988 81.915) (width 0.25) (layer B.Cu) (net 2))
 (segment (start 165.608 83.185) (end 159.258 83.185) (width 0.25) (layer B.Cu) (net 2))
 (segment (start 157.988 81.915) (end 157.988 90.805) (width 0.25) (layer B.Cu) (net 2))
 (segment (start 156.998051 90.805) (end 157.988 90.805) (width 0.25) (layer F.Cu) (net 2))
 (segment (start 142.995002 90.805) (end 156.998051 90.805) (width 0.25) (layer F.Cu) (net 2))
 (segment (start 141.970001 91.830001) (end 142.995002 90.805) (width 0.25) (layer F.Cu) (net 2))
 (segment (start 136.462999 91.830001) (end 141.970001 91.830001) (width 0.25) (layer F.Cu) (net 2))
 (segment (start 128.778 99.515) (end 136.462999 91.830001) (width 0.25) (layer F.Cu) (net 2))
 (segment (start 128.778 100.965) (end 128.778 99.515) (width 0.25) (layer F.Cu) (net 2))
 (segment (start 170.688 95.885) (end 165.608 90.805) (width 0.25) (layer B.Cu) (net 1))
 (segment (start 167.108 89.305) (end 167.108 83.185) (width 0.25) (layer B.Cu) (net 1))
 (segment (start 165.608 90.805) (end 167.108 89.305) (width 0.25) (layer B.Cu) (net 1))
 (segment (start 164.582999 91.830001) (end 164.908001 91.504999) (width 0.25) (layer F.Cu) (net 1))
 (segment (start 153.852997 91.830001) (end 164.582999 91.830001) (width 0.25) (layer F.Cu) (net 1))
 (segment (start 164.908001 91.504999) (end 165.608 90.805) (width 0.25) (layer F.Cu) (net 1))
 (segment (start 143.192997 102.490001) (end 153.852997 91.830001) (width 0.25) (layer F.Cu) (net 1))
 (segment (start 130.882999 102.490001) (end 143.192997 102.490001) (width 0.25) (layer F.Cu) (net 1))
 (segment (start 126.238 107.135) (end 130.882999 102.490001) (width 0.25) (layer F.Cu) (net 1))
 (segment (start 126.238 108.585) (end 126.238 107.135) (width 0.25) (layer F.Cu) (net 1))
 (segment (start 126.238 97.155) (end 128.778 94.615) (width 0.25) (layer B.Cu) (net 4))
 (segment (start 126.238 100.965) (end 126.238 97.155) (width 0.25) (layer B.Cu) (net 4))
 (segment (start 142.467949 90.805) (end 141.478 90.805) (width 0.25) (layer B.Cu) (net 4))
 (segment (start 149.948 90.805) (end 142.467949 90.805) (width 0.25) (layer B.Cu) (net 4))
 (segment (start 151.638 89.115) (end 149.948 90.805) (width 0.25) (layer B.Cu) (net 4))
 (segment (start 151.638 88.265) (end 151.638 89.115) (width 0.25) (layer B.Cu) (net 4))
 (segment (start 128.778 94.615) (end 128.778 92.075) (width 0.25) (layer B.Cu) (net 4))
 (segment (start 128.778 92.075) (end 131.318 89.535) (width 0.25) (layer B.Cu) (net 4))
 (segment (start 140.208 89.535) (end 141.478 90.805) (width 0.25) (layer B.Cu) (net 4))
 (segment (start 131.318 89.535) (end 140.208 89.535) (width 0.25) (layer B.Cu) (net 4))
 (segment (start 152.70567 104.921087) (end 152.70567 104.799861) (width 0.25) (layer F.Cu) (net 10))
 (segment (start 156.813579 105.937086) (end 153.721669 105.937086) (width 0.25) (layer F.Cu) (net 10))
 (segment (start 161.798 100.952665) (end 156.813579 105.937086) (width 0.25) (layer F.Cu) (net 10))
 (segment (start 152.70567 104.799861) (end 152.70567 103.951333) (width 0.25) (layer F.Cu) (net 10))
 (segment (start 153.721669 105.937086) (end 152.70567 104.921087) (width 0.25) (layer F.Cu) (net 10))
 (segment (start 161.798 96.615) (end 161.798 100.952665) (width 0.25) (layer F.Cu) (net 10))
 (segment (start 157.43033 99.670139) (end 157.43033 100.518667) (width 0.25) (layer B.Cu) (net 12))
 (segment (start 157.43033 98.30767) (end 157.43033 99.670139) (width 0.25) (layer B.Cu) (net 12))
 (segment (start 161.123 94.615) (end 157.43033 98.30767) (width 0.25) (layer B.Cu) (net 12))
 (segment (start 161.798 94.615) (end 161.123 94.615) (width 0.25) (layer B.Cu) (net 12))
 (segment (start 147.335085 99.457915) (end 154.16567 99.457915) (width 0.25) (layer B.Cu) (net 6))
 (segment (start 145.288 101.505) (end 147.335085 99.457915) (width 0.25) (layer B.Cu) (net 6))
 (segment (start 144.288 102.505) (end 145.288 102.505) (width 0.25) (layer B.Cu) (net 7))
 (segment (start 136.398 94.615) (end 144.288 102.505) (width 0.25) (layer B.Cu) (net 7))
 (segment (start 145.288 103.505) (end 145.288 106.045) (width 0.25) (layer F.Cu) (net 8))
 (segment (start 145.288 106.045) (end 150.368 111.125) (width 0.25) (layer F.Cu) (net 8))
 (segment (start 150.368 111.125) (end 150.368 111.125) (width 0.25) (layer F.Cu) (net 8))
 (via (at 150.368 111.125) (size 0.6) (drill 0.4) (layers F.Cu B.Cu) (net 8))
 (segment (start 150.368 111.125) (end 154.178 111.125) (width 0.25) (layer B.Cu) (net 8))
 (segment (start 155.97033 109.33267) (end 155.97033 105.012085) (width 0.25) (layer B.Cu) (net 8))
 (segment (start 154.178 111.125) (end 155.97033 109.33267) (width 0.25) (layer B.Cu) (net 8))
 (segment (start 114.492594 99.155) (end 115.222594 98.425) (width 0.25) (layer F.Cu) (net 19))
 (segment (start 113.538 99.155) (end 114.492594 99.155) (width 0.25) (layer F.Cu) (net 19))
 (segment (start 115.222594 98.425) (end 119.888 98.425) (width 0.25) (layer F.Cu) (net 19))
 (segment (start 115.222594 98.425) (end 121.158 98.425) (width 0.25) (layer F.Cu) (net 19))
 (segment (start 121.158 98.425) (end 133.858 85.725) (width 0.25) (layer F.Cu) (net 19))
 (segment (start 145.034 76.831) (end 145.034 75.565) (width 0.25) (layer F.Cu) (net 19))
 (segment (start 136.14 85.725) (end 145.034 76.831) (width 0.25) (layer F.Cu) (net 19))
 (segment (start 133.858 85.725) (end 136.14 85.725) (width 0.25) (layer F.Cu) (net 19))
 (segment (start 113.538 97.155) (end 117.348 97.155) (width 0.25) (layer B.Cu) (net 20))
 (segment (start 117.348 97.155) (end 126.238 88.265) (width 0.25) (layer B.Cu) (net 20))
 (segment (start 126.238 88.265) (end 126.238 83.185) (width 0.25) (layer B.Cu) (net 20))
 (segment (start 126.238 83.185) (end 130.048 79.375) (width 0.25) (layer B.Cu) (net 20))
 (segment (start 147.574 76.831) (end 147.574 75.565) (width 0.25) (layer B.Cu) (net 20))
 (segment (start 145.03 79.375) (end 147.574 76.831) (width 0.25) (layer B.Cu) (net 20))
 (segment (start 130.048 79.375) (end 145.03 79.375) (width 0.25) (layer B.Cu) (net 20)))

